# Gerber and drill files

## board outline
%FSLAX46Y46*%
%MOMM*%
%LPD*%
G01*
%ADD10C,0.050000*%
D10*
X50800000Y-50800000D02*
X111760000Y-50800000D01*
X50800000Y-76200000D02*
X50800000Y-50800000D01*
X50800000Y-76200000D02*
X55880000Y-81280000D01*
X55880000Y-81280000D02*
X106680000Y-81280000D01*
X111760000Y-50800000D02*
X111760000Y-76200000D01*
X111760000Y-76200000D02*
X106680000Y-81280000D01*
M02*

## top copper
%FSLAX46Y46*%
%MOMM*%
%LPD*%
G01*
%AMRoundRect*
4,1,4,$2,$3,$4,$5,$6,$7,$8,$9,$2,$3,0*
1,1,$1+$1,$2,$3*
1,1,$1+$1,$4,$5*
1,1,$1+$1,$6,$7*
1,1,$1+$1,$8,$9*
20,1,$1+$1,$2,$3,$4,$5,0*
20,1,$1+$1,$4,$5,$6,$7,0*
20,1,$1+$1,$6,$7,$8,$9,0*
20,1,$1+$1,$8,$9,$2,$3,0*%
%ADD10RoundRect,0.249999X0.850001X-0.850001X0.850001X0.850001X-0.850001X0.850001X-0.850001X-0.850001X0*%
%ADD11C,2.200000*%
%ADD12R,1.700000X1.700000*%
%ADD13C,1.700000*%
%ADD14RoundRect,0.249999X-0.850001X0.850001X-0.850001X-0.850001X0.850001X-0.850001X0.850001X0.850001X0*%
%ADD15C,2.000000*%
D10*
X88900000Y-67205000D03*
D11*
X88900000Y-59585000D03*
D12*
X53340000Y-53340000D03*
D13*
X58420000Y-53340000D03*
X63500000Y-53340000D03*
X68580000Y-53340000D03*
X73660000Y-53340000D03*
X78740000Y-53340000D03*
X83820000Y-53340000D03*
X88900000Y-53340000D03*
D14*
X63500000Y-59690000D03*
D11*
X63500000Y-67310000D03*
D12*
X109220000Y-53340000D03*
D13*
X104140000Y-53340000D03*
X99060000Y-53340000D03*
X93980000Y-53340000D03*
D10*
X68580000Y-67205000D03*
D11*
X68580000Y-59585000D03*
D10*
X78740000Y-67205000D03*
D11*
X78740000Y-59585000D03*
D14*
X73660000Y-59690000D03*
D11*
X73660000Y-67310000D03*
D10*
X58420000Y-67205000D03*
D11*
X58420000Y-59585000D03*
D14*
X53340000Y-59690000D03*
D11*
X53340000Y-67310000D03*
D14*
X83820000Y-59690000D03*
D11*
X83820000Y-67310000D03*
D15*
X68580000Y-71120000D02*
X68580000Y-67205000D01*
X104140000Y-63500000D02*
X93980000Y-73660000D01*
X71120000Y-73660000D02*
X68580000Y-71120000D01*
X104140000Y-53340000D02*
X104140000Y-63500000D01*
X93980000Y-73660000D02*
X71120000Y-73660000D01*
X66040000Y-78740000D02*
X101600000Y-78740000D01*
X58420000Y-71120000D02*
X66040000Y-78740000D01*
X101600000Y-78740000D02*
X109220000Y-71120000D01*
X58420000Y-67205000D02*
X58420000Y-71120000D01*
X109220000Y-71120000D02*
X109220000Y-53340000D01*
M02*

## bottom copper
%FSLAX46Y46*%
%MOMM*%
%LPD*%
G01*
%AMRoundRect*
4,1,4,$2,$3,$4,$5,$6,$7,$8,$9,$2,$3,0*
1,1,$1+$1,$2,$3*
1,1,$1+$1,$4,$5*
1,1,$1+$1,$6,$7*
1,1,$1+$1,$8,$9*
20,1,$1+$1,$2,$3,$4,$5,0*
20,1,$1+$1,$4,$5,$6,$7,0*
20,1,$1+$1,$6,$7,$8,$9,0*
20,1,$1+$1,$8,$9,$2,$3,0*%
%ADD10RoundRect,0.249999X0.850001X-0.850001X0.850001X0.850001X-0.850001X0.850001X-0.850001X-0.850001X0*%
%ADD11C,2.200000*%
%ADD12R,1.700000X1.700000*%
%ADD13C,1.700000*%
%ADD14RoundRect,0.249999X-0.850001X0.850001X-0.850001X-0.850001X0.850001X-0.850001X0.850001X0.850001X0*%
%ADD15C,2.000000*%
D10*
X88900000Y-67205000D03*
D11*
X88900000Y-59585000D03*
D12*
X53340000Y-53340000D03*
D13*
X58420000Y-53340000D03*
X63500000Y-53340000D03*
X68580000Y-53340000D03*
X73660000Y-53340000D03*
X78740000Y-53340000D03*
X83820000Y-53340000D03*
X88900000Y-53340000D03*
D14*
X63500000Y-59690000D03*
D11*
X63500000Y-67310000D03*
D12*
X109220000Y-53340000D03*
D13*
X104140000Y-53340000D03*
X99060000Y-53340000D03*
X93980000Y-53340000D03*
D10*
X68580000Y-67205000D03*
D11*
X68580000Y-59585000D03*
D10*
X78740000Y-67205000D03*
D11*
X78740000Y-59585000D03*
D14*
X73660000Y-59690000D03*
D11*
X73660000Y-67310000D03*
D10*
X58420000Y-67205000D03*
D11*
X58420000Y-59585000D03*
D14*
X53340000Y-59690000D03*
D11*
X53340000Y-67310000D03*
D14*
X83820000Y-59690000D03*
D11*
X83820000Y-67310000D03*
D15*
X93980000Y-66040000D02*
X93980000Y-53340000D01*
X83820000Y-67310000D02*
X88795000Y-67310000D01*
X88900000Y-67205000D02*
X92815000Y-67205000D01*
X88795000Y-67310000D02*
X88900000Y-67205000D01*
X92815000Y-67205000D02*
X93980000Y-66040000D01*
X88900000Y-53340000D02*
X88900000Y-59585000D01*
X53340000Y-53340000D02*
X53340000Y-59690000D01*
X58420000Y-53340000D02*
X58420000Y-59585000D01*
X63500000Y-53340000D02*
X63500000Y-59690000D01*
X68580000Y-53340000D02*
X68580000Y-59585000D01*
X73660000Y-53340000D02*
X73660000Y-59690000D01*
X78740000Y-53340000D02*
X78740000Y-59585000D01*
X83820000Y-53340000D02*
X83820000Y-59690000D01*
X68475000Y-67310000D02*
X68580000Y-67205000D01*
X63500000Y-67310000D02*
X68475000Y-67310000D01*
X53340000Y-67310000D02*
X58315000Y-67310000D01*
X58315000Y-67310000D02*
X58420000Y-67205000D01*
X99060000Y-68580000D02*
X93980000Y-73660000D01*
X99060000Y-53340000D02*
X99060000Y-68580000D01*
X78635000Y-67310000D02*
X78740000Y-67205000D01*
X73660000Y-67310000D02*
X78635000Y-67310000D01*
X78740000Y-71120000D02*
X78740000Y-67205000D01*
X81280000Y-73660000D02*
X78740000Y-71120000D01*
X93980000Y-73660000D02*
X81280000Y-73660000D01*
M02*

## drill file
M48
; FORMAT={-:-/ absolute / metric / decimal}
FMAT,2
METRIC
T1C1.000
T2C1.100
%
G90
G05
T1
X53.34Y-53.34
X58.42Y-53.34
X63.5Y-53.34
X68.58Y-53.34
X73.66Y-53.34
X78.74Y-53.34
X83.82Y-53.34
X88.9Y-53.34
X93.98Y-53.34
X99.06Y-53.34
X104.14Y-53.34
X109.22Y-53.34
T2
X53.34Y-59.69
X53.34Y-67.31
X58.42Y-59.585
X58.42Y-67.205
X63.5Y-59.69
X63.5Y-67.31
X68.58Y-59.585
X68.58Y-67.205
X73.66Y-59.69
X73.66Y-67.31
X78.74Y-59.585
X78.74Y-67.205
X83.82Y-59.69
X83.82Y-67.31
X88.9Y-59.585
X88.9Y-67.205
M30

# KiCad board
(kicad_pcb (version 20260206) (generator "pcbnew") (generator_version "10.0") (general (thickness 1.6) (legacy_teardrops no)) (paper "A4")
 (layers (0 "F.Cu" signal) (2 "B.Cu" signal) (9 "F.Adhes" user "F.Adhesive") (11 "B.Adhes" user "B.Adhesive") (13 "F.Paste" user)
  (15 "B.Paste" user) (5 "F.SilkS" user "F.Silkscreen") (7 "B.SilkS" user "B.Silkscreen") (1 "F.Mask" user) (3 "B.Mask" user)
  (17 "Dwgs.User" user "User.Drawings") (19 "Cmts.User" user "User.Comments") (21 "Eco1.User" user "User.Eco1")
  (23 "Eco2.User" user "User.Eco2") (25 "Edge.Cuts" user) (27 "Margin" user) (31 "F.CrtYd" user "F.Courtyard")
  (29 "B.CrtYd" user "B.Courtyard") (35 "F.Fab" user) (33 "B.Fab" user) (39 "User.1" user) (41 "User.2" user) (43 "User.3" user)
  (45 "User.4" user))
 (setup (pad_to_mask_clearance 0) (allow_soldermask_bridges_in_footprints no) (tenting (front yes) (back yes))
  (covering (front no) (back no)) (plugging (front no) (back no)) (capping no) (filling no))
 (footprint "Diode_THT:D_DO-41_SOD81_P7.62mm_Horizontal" (layer "F.Cu") (at 88.9 67.205 90)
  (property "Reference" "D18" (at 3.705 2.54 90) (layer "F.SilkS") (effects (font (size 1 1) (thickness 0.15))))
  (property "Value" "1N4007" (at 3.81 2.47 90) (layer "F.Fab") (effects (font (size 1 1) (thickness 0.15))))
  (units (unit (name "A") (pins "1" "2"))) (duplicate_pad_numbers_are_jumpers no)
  (pad "1" thru_hole roundrect (at 0 0 90) (size 2.2 2.2) (drill 1.1) (layers "*.Cu" "*.Mask") (remove_unused_layers no)
   (roundrect_rratio 0.113636) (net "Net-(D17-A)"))
  (pad "2" thru_hole circle (at 7.62 0 90) (size 2.2 2.2) (drill 1.1) (layers "*.Cu" "*.Mask") (remove_unused_layers no) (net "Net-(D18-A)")))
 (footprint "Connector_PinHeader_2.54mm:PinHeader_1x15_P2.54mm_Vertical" (layer "F.Cu") (at 53.34 53.34 90)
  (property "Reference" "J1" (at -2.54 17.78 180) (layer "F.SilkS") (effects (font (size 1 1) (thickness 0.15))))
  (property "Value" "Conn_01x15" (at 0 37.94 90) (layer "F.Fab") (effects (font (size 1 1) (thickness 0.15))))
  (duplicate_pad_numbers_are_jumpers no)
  (pad "1" thru_hole rect (at 0 0 90) (size 1.7 1.7) (drill 1) (layers "*.Cu" "*.Mask") (remove_unused_layers no) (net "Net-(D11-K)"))
  (pad "3" thru_hole circle (at 0 5.08 90) (size 1.7 1.7) (drill 1) (layers "*.Cu" "*.Mask") (remove_unused_layers no) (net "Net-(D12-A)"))
  (pad "5" thru_hole circle (at 0 10.16 90) (size 1.7 1.7) (drill 1) (layers "*.Cu" "*.Mask") (remove_unused_layers no) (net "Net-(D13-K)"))
  (pad "7" thru_hole circle (at 0 15.24 90) (size 1.7 1.7) (drill 1) (layers "*.Cu" "*.Mask") (remove_unused_layers no) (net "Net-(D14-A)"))
  (pad "9" thru_hole circle (at 0 20.32 90) (size 1.7 1.7) (drill 1) (layers "*.Cu" "*.Mask") (remove_unused_layers no) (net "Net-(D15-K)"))
  (pad "11" thru_hole circle (at 0 25.4 90) (size 1.7 1.7) (drill 1) (layers "*.Cu" "*.Mask") (remove_unused_layers no) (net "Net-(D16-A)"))
  (pad "13" thru_hole circle (at 0 30.48 90) (size 1.7 1.7) (drill 1) (layers "*.Cu" "*.Mask") (remove_unused_layers no) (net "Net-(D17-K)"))
  (pad "15" thru_hole circle (at 0 35.56 90) (size 1.7 1.7) (drill 1) (layers "*.Cu" "*.Mask") (remove_unused_layers no) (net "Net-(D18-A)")))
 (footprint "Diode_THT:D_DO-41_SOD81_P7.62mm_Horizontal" (layer "F.Cu") (at 63.5 59.69 -90)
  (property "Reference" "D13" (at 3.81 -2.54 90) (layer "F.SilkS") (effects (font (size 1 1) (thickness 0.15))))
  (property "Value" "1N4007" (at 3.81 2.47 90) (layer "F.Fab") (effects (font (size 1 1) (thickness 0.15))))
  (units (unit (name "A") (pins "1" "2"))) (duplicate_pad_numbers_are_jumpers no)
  (pad "1" thru_hole roundrect (at 0 0 270) (size 2.2 2.2) (drill 1.1) (layers "*.Cu" "*.Mask") (remove_unused_layers no)
   (roundrect_rratio 0.113636) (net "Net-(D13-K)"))
  (pad "2" thru_hole circle (at 7.62 0 270) (size 2.2 2.2) (drill 1.1) (layers "*.Cu" "*.Mask") (remove_unused_layers no)
   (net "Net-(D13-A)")))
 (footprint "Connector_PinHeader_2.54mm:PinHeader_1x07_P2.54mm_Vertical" (layer "F.Cu") (at 109.22 53.34 -90)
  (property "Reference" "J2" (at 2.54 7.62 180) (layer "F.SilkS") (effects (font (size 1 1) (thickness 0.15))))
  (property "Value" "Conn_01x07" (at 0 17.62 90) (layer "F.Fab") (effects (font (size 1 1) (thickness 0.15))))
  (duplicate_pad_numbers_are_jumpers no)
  (pad "1" thru_hole rect (at 0 0 270) (size 1.7 1.7) (drill 1) (layers "*.Cu" "*.Mask") (remove_unused_layers no) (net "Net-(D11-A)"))
  (pad "3" thru_hole circle (at 0 5.08 270) (size 1.7 1.7) (drill 1) (layers "*.Cu" "*.Mask") (remove_unused_layers no) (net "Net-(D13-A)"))
  (pad "5" thru_hole circle (at 0 10.16 270) (size 1.7 1.7) (drill 1) (layers "*.Cu" "*.Mask") (remove_unused_layers no) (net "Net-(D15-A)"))
  (pad "7" thru_hole circle (at 0 15.24 270) (size 1.7 1.7) (drill 1) (layers "*.Cu" "*.Mask") (remove_unused_layers no) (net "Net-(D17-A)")))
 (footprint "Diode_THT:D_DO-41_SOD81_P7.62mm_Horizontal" (layer "F.Cu") (at 68.58 67.205 90)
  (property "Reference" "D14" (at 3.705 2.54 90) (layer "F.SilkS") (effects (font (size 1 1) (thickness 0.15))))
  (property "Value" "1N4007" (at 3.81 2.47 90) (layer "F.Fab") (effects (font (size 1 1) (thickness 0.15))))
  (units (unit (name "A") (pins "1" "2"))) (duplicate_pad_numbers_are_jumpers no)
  (pad "1" thru_hole roundrect (at 0 0 90) (size 2.2 2.2) (drill 1.1) (layers "*.Cu" "*.Mask") (remove_unused_layers no)
   (roundrect_rratio 0.113636) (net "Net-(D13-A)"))
  (pad "2" thru_hole circle (at 7.62 0 90) (size 2.2 2.2) (drill 1.1) (layers "*.Cu" "*.Mask") (remove_unused_layers no) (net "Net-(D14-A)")))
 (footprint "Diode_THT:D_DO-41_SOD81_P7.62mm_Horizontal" (layer "F.Cu") (at 78.74 67.205 90)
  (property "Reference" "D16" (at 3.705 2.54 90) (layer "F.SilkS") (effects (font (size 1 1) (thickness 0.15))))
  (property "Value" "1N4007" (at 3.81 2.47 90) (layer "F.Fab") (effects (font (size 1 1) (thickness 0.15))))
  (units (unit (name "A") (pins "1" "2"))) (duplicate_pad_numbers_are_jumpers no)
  (pad "1" thru_hole roundrect (at 0 0 90) (size 2.2 2.2) (drill 1.1) (layers "*.Cu" "*.Mask") (remove_unused_layers no)
   (roundrect_rratio 0.113636) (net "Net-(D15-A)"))
  (pad "2" thru_hole circle (at 7.62 0 90) (size 2.2 2.2) (drill 1.1) (layers "*.Cu" "*.Mask") (remove_unused_layers no) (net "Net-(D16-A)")))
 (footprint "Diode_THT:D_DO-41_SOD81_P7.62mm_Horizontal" (layer "F.Cu") (at 73.66 59.69 -90)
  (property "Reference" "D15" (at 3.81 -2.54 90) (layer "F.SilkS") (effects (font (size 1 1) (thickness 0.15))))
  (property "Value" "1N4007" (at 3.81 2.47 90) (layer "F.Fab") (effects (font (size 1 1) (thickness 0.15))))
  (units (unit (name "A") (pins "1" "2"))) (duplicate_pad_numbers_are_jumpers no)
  (pad "1" thru_hole roundrect (at 0 0 270) (size 2.2 2.2) (drill 1.1) (layers "*.Cu" "*.Mask") (remove_unused_layers no)
   (roundrect_rratio 0.113636) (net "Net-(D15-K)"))
  (pad "2" thru_hole circle (at 7.62 0 270) (size 2.2 2.2) (drill 1.1) (layers "*.Cu" "*.Mask") (remove_unused_layers no)
   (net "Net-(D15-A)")))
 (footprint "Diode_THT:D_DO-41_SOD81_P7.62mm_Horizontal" (layer "F.Cu") (at 58.42 67.205 90)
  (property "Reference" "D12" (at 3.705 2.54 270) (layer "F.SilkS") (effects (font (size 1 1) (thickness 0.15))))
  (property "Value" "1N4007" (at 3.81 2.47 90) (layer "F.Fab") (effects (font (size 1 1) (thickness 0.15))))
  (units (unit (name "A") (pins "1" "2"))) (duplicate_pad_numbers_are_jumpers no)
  (pad "1" thru_hole roundrect (at 0 0 90) (size 2.2 2.2) (drill 1.1) (layers "*.Cu" "*.Mask") (remove_unused_layers no)
   (roundrect_rratio 0.113636) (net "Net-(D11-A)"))
  (pad "2" thru_hole circle (at 7.62 0 90) (size 2.2 2.2) (drill 1.1) (layers "*.Cu" "*.Mask") (remove_unused_layers no) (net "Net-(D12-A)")))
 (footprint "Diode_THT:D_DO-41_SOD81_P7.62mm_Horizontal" (layer "F.Cu") (at 53.34 59.69 -90)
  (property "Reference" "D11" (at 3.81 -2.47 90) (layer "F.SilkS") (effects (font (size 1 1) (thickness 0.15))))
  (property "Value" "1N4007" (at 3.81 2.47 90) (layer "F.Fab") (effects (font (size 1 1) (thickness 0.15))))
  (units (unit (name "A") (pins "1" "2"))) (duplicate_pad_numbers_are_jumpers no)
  (pad "1" thru_hole roundrect (at 0 0 270) (size 2.2 2.2) (drill 1.1) (layers "*.Cu" "*.Mask") (remove_unused_layers no)
   (roundrect_rratio 0.113636) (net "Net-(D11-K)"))
  (pad "2" thru_hole circle (at 7.62 0 270) (size 2.2 2.2) (drill 1.1) (layers "*.Cu" "*.Mask") (remove_unused_layers no)
   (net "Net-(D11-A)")))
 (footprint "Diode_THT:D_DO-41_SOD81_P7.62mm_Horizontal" (layer "F.Cu") (at 83.82 59.69 -90)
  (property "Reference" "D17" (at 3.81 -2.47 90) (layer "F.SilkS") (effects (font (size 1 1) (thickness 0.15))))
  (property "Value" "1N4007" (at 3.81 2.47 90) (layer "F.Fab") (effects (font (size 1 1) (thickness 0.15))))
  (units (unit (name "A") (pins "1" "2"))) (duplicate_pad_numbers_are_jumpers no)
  (pad "1" thru_hole roundrect (at 0 0 270) (size 2.2 2.2) (drill 1.1) (layers "*.Cu" "*.Mask") (remove_unused_layers no)
   (roundrect_rratio 0.113636) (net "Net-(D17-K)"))
  (pad "2" thru_hole circle (at 7.62 0 270) (size 2.2 2.2) (drill 1.1) (layers "*.Cu" "*.Mask") (remove_unused_layers no)
   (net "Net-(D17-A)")))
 (gr_line (start 50.8 50.8) (end 111.76 50.8) (stroke (width 0.05) (type default)) (layer "Edge.Cuts"))
 (gr_line (start 50.8 76.2) (end 50.8 50.8) (stroke (width 0.05) (type default)) (layer "Edge.Cuts"))
 (gr_line (start 50.8 76.2) (end 55.88 81.28) (stroke (width 0.05) (type default)) (layer "Edge.Cuts"))
 (gr_line (start 55.88 81.28) (end 106.68 81.28) (stroke (width 0.05) (type default)) (layer "Edge.Cuts"))
 (gr_line (start 111.76 50.8) (end 111.76 76.2) (stroke (width 0.05) (type default)) (layer "Edge.Cuts"))
 (gr_line (start 111.76 76.2) (end 106.68 81.28) (stroke (width 0.05) (type default)) (layer "Edge.Cuts"))
 (segment (start 93.98 66.04) (end 93.98 53.34) (width 2) (layer "B.Cu") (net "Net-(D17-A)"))
 (segment (start 83.82 67.31) (end 88.795 67.31) (width 2) (layer "B.Cu") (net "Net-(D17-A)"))
 (segment (start 88.9 67.205) (end 92.815 67.205) (width 2) (layer "B.Cu") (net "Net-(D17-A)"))
 (segment (start 88.795 67.31) (end 88.9 67.205) (width 2) (layer "B.Cu") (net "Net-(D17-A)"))
 (segment (start 92.815 67.205) (end 93.98 66.04) (width 2) (layer "B.Cu") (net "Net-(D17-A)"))
 (segment (start 88.9 53.34) (end 88.9 59.585) (width 2) (layer "B.Cu") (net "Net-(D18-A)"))
 (segment (start 53.34 53.34) (end 53.34 59.69) (width 2) (layer "B.Cu") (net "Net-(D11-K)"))
 (segment (start 58.42 53.34) (end 58.42 59.585) (width 2) (layer "B.Cu") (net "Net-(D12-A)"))
 (segment (start 63.5 53.34) (end 63.5 59.69) (width 2) (layer "B.Cu") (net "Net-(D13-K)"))
 (segment (start 68.58 53.34) (end 68.58 59.585) (width 2) (layer "B.Cu") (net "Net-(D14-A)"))
 (segment (start 73.66 53.34) (end 73.66 59.69) (width 2) (layer "B.Cu") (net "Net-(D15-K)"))
 (segment (start 78.74 53.34) (end 78.74 59.585) (width 2) (layer "B.Cu") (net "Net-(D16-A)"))
 (segment (start 83.82 53.34) (end 83.82 59.69) (width 2) (layer "B.Cu") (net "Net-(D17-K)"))
 (segment (start 68.58 71.12) (end 68.58 67.205) (width 2) (layer "F.Cu") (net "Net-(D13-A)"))
 (segment (start 104.14 63.5) (end 93.98 73.66) (width 2) (layer "F.Cu") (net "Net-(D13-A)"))
 (segment (start 71.12 73.66) (end 68.58 71.12) (width 2) (layer "F.Cu") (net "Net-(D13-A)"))
 (segment (start 104.14 53.34) (end 104.14 63.5) (width 2) (layer "F.Cu") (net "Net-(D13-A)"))
 (segment (start 93.98 73.66) (end 71.12 73.66) (width 2) (layer "F.Cu") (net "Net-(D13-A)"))
 (segment (start 68.475 67.31) (end 68.58 67.205) (width 2) (layer "B.Cu") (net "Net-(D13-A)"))
 (segment (start 63.5 67.31) (end 68.475 67.31) (width 2) (layer "B.Cu") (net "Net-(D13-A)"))
 (segment (start 66.04 78.74) (end 101.6 78.74) (width 2) (layer "F.Cu") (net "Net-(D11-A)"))
 (segment (start 58.42 71.12) (end 66.04 78.74) (width 2) (layer "F.Cu") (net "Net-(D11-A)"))
 (segment (start 101.6 78.74) (end 109.22 71.12) (width 2) (layer "F.Cu") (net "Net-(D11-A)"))
 (segment (start 58.42 67.205) (end 58.42 71.12) (width 2) (layer "F.Cu") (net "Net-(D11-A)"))
 (segment (start 109.22 71.12) (end 109.22 53.34) (width 2) (layer "F.Cu") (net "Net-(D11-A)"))
 (segment (start 53.34 67.31) (end 58.315 67.31) (width 2) (layer "B.Cu") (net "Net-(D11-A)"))
 (segment (start 58.315 67.31) (end 58.42 67.205) (width 2) (layer "B.Cu") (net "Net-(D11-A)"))
 (segment (start 99.06 68.58) (end 93.98 73.66) (width 2) (layer "B.Cu") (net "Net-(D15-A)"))
 (segment (start 99.06 53.34) (end 99.06 68.58) (width 2) (layer "B.Cu") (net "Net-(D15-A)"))
 (segment (start 78.635 67.31) (end 78.74 67.205) (width 2) (layer "B.Cu") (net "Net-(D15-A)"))
 (segment (start 73.66 67.31) (end 78.635 67.31) (width 2) (layer "B.Cu") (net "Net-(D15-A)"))
 (segment (start 78.74 71.12) (end 78.74 67.205) (width 2) (layer "B.Cu") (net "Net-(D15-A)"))
 (segment (start 81.28 73.66) (end 78.74 71.12) (width 2) (layer "B.Cu") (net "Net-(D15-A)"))
 (segment (start 93.98 73.66) (end 81.28 73.66) (width 2) (layer "B.Cu") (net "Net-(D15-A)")))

